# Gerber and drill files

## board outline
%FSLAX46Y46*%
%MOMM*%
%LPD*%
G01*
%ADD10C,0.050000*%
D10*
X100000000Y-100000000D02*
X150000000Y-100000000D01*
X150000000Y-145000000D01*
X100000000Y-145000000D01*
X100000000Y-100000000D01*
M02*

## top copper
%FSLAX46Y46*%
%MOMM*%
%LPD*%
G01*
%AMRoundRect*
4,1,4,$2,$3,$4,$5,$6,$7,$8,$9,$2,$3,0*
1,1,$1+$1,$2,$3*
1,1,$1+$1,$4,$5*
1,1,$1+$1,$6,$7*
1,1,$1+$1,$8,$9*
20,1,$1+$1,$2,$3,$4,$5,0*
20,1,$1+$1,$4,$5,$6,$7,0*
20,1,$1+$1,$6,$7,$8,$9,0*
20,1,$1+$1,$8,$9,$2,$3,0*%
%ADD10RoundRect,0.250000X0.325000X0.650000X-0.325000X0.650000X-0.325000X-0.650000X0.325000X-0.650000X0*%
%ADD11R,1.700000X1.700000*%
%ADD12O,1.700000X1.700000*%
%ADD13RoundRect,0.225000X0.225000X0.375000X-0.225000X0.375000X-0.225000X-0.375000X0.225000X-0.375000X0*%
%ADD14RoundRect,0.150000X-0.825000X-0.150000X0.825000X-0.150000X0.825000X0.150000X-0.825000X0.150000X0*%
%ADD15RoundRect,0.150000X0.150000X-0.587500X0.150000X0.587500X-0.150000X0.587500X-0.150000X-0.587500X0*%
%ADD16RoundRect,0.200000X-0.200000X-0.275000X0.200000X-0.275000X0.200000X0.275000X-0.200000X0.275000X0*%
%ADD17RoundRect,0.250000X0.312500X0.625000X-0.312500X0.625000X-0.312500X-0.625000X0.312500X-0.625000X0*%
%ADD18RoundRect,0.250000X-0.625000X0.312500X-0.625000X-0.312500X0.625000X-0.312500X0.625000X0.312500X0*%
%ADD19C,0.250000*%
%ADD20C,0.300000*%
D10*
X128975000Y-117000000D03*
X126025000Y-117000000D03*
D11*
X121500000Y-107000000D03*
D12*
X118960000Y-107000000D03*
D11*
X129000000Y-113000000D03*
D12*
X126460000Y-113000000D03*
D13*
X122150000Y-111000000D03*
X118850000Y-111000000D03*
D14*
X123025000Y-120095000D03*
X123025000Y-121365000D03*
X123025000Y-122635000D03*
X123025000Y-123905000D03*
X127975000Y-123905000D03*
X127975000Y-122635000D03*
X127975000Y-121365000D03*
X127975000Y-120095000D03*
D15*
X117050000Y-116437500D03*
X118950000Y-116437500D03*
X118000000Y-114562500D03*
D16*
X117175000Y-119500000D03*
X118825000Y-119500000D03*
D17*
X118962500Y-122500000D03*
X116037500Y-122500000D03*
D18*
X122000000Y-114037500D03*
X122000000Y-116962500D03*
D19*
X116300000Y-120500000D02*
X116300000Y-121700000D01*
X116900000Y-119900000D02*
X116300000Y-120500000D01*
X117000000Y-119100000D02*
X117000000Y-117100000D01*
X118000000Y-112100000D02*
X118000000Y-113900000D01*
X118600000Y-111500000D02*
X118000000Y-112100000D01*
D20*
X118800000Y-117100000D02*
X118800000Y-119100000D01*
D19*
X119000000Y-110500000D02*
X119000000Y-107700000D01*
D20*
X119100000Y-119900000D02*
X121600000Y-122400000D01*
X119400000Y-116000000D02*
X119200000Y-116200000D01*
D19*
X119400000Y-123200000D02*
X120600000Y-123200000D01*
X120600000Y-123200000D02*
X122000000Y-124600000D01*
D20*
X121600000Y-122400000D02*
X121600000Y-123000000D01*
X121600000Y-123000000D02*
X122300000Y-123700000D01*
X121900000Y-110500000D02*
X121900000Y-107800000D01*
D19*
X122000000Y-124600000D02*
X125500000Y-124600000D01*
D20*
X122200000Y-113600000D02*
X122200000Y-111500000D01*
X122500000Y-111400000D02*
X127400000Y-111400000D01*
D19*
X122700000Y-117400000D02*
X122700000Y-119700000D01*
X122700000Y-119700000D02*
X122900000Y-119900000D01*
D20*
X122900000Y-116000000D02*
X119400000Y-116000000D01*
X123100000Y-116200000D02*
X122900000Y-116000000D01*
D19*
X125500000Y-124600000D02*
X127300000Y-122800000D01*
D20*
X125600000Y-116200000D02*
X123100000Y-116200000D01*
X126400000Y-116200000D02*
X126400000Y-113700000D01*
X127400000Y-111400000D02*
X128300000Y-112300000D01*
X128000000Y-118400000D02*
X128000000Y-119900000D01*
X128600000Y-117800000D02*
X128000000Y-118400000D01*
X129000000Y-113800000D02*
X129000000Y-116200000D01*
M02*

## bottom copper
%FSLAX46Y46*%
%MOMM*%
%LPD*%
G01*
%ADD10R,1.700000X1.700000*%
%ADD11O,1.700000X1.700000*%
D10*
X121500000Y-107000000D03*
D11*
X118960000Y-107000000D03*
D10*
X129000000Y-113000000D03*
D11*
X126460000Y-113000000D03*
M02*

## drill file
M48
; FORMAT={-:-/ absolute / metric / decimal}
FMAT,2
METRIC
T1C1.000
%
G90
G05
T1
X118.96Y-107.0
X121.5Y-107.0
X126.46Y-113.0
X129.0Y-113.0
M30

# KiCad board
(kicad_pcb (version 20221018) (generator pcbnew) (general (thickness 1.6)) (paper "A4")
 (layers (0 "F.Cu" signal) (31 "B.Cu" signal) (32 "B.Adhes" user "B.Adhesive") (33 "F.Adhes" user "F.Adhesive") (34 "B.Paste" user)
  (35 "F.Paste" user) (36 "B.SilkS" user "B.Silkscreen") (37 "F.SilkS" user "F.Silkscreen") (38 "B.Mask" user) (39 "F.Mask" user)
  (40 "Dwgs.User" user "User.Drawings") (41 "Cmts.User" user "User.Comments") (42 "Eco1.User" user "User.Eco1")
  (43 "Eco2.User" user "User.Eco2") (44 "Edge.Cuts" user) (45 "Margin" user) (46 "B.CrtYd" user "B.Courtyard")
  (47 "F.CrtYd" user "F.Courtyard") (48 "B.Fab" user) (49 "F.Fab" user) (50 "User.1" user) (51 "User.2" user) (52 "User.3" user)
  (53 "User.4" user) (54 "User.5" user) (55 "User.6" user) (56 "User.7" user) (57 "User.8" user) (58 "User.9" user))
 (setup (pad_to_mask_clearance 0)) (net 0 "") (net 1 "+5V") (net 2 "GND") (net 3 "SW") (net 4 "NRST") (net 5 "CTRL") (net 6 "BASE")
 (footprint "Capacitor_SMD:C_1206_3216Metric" (layer "F.Cu") (at 127.5 117 180)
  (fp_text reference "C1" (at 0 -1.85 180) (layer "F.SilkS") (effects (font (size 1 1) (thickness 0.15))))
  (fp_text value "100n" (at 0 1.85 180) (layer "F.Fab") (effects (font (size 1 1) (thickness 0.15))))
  (pad "1" smd roundrect (at -1.475 0 180) (size 1.15 1.8) (layers "F.Cu" "F.Paste" "F.Mask") (roundrect_rratio 0.217391) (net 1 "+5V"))
  (pad "2" smd roundrect (at 1.475 0 180) (size 1.15 1.8) (layers "F.Cu" "F.Paste" "F.Mask") (roundrect_rratio 0.217391) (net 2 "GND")))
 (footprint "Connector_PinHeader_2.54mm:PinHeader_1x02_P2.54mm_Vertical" (layer "F.Cu") (at 121.5 107 -90)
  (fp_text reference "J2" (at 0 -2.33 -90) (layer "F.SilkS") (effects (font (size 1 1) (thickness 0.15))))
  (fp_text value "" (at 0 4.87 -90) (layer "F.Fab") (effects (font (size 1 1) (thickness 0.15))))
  (pad "1" thru_hole rect (at 0 0 270) (size 1.7 1.7) (drill 1) (layers "*.Cu" "*.Mask") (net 1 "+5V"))
  (pad "2" thru_hole oval (at 0 2.54 270) (size 1.7 1.7) (drill 1) (layers "*.Cu" "*.Mask") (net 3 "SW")))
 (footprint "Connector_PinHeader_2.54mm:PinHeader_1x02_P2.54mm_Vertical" (layer "F.Cu") (at 129 113 -90)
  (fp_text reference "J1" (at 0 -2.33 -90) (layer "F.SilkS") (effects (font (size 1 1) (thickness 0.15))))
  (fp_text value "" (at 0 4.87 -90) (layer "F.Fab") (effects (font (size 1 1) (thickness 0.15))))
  (pad "1" thru_hole rect (at 0 0 270) (size 1.7 1.7) (drill 1) (layers "*.Cu" "*.Mask") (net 1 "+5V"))
  (pad "2" thru_hole oval (at 0 2.54 270) (size 1.7 1.7) (drill 1) (layers "*.Cu" "*.Mask") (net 2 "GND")))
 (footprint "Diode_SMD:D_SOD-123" (layer "F.Cu") (at 120.5 111 180)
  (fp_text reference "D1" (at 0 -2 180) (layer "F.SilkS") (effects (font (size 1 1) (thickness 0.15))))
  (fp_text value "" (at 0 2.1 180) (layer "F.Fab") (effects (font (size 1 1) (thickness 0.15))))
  (pad "1" smd roundrect (at -1.65 0 180) (size 0.9 1.2) (layers "F.Cu" "F.Paste" "F.Mask") (roundrect_rratio 0.25) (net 1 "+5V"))
  (pad "2" smd roundrect (at 1.65 0 180) (size 0.9 1.2) (layers "F.Cu" "F.Paste" "F.Mask") (roundrect_rratio 0.25) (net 3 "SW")))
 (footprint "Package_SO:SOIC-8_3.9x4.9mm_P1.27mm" (layer "F.Cu") (at 125.5 122)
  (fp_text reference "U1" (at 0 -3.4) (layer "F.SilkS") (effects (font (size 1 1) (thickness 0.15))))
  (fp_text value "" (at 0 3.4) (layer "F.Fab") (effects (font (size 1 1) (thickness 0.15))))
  (pad "1" smd roundrect (at -2.475 -1.905) (size 1.95 0.6) (layers "F.Cu" "F.Paste" "F.Mask") (roundrect_rratio 0.25) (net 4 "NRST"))
  (pad "2" smd roundrect (at -2.475 -0.635) (size 1.95 0.6) (layers "F.Cu" "F.Paste" "F.Mask") (roundrect_rratio 0.25))
  (pad "3" smd roundrect (at -2.475 0.635) (size 1.95 0.6) (layers "F.Cu" "F.Paste" "F.Mask") (roundrect_rratio 0.25))
  (pad "4" smd roundrect (at -2.475 1.905) (size 1.95 0.6) (layers "F.Cu" "F.Paste" "F.Mask") (roundrect_rratio 0.25) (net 2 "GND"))
  (pad "5" smd roundrect (at 2.475 1.905) (size 1.95 0.6) (layers "F.Cu" "F.Paste" "F.Mask") (roundrect_rratio 0.25))
  (pad "6" smd roundrect (at 2.475 0.635) (size 1.95 0.6) (layers "F.Cu" "F.Paste" "F.Mask") (roundrect_rratio 0.25) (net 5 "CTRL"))
  (pad "7" smd roundrect (at 2.475 -0.635) (size 1.95 0.6) (layers "F.Cu" "F.Paste" "F.Mask") (roundrect_rratio 0.25))
  (pad "8" smd roundrect (at 2.475 -1.905) (size 1.95 0.6) (layers "F.Cu" "F.Paste" "F.Mask") (roundrect_rratio 0.25) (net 1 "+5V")))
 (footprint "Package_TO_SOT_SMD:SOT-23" (layer "F.Cu") (at 118 115.5 90)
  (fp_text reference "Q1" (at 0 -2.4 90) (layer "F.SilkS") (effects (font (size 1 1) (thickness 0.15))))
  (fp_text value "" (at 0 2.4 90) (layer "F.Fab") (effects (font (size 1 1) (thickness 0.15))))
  (pad "1" smd roundrect (at -0.9375 -0.95 90) (size 1.475 0.6) (layers "F.Cu" "F.Paste" "F.Mask") (roundrect_rratio 0.25) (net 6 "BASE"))
  (pad "2" smd roundrect (at -0.9375 0.95 90) (size 1.475 0.6) (layers "F.Cu" "F.Paste" "F.Mask") (roundrect_rratio 0.25) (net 2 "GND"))
  (pad "3" smd roundrect (at 0.9375 0 90) (size 1.475 0.6) (layers "F.Cu" "F.Paste" "F.Mask") (roundrect_rratio 0.25) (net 3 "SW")))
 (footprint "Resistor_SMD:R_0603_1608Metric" (layer "F.Cu") (at 118 119.5)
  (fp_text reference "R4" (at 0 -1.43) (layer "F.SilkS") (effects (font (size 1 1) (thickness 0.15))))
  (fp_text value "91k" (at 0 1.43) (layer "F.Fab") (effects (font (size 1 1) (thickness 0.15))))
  (pad "1" smd roundrect (at -0.825 0) (size 0.8 0.95) (layers "F.Cu" "F.Paste" "F.Mask") (roundrect_rratio 0.25) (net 6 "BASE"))
  (pad "2" smd roundrect (at 0.825 0) (size 0.8 0.95) (layers "F.Cu" "F.Paste" "F.Mask") (roundrect_rratio 0.25) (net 2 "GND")))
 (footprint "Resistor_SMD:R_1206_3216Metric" (layer "F.Cu") (at 117.5 122.5 180)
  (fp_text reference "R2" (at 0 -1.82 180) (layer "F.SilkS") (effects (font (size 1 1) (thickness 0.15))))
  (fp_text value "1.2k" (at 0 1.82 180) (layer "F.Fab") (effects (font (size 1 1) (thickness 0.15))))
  (pad "1" smd roundrect (at -1.4625 0 180) (size 1.125 1.75) (layers "F.Cu" "F.Paste" "F.Mask") (roundrect_rratio 0.222222) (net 5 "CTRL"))
  (pad "2" smd roundrect (at 1.4625 0 180) (size 1.125 1.75) (layers "F.Cu" "F.Paste" "F.Mask") (roundrect_rratio 0.222222) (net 6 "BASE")))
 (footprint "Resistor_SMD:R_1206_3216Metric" (layer "F.Cu") (at 122 115.5 -90)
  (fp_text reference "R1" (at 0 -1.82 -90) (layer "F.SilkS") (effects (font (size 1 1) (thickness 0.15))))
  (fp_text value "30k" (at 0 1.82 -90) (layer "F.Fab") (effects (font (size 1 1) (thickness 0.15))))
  (pad "1" smd roundrect (at -1.4625 0 270) (size 1.125 1.75) (layers "F.Cu" "F.Paste" "F.Mask") (roundrect_rratio 0.222222) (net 1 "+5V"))
  (pad "2" smd roundrect (at 1.4625 0 270) (size 1.125 1.75) (layers "F.Cu" "F.Paste" "F.Mask") (roundrect_rratio 0.222222) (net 4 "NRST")))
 (gr_rect (start 100 100) (end 150 145) (stroke (width 0.05) (type default)) (fill none) (layer "Edge.Cuts"))
 (segment (start 116.3 120.5) (end 116.3 121.7) (width 0.25) (layer "F.Cu") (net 6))
 (segment (start 116.9 119.9) (end 116.3 120.5) (width 0.25) (layer "F.Cu") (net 6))
 (segment (start 117 119.1) (end 117 117.1) (width 0.25) (layer "F.Cu") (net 6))
 (segment (start 118 112.1) (end 118 113.9) (width 0.25) (layer "F.Cu") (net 3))
 (segment (start 118.6 111.5) (end 118 112.1) (width 0.25) (layer "F.Cu") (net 3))
 (segment (start 118.8 117.1) (end 118.8 119.1) (width 0.3) (layer "F.Cu") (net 2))
 (segment (start 119 110.5) (end 119 107.7) (width 0.25) (layer "F.Cu") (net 3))
 (segment (start 119.1 119.9) (end 121.6 122.4) (width 0.3) (layer "F.Cu") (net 2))
 (segment (start 119.4 116) (end 119.2 116.2) (width 0.3) (layer "F.Cu") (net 2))
 (segment (start 119.4 123.2) (end 120.6 123.2) (width 0.25) (layer "F.Cu") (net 5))
 (segment (start 120.6 123.2) (end 122 124.6) (width 0.25) (layer "F.Cu") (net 5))
 (segment (start 121.6 122.4) (end 121.6 123) (width 0.3) (layer "F.Cu") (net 2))
 (segment (start 121.6 123) (end 122.3 123.7) (width 0.3) (layer "F.Cu") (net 2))
 (segment (start 121.9 110.5) (end 121.9 107.8) (width 0.3) (layer "F.Cu") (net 1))
 (segment (start 122 124.6) (end 125.5 124.6) (width 0.25) (layer "F.Cu") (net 5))
 (segment (start 122.2 113.6) (end 122.2 111.5) (width 0.3) (layer "F.Cu") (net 1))
 (segment (start 122.5 111.4) (end 127.4 111.4) (width 0.3) (layer "F.Cu") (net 1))
 (segment (start 122.7 117.4) (end 122.7 119.7) (width 0.25) (layer "F.Cu") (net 4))
 (segment (start 122.7 119.7) (end 122.9 119.9) (width 0.25) (layer "F.Cu") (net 4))
 (segment (start 122.9 116) (end 119.4 116) (width 0.3) (layer "F.Cu") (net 2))
 (segment (start 123.1 116.2) (end 122.9 116) (width 0.3) (layer "F.Cu") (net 2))
 (segment (start 125.5 124.6) (end 127.3 122.8) (width 0.25) (layer "F.Cu") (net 5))
 (segment (start 125.6 116.2) (end 123.1 116.2) (width 0.3) (layer "F.Cu") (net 2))
 (segment (start 126.4 116.2) (end 126.4 113.7) (width 0.3) (layer "F.Cu") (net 2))
 (segment (start 127.4 111.4) (end 128.3 112.3) (width 0.3) (layer "F.Cu") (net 1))
 (segment (start 128 118.4) (end 128 119.9) (width 0.3) (layer "F.Cu") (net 1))
 (segment (start 128.6 117.8) (end 128 118.4) (width 0.3) (layer "F.Cu") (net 1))
 (segment (start 129 113.8) (end 129 116.2) (width 0.3) (layer "F.Cu") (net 1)))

